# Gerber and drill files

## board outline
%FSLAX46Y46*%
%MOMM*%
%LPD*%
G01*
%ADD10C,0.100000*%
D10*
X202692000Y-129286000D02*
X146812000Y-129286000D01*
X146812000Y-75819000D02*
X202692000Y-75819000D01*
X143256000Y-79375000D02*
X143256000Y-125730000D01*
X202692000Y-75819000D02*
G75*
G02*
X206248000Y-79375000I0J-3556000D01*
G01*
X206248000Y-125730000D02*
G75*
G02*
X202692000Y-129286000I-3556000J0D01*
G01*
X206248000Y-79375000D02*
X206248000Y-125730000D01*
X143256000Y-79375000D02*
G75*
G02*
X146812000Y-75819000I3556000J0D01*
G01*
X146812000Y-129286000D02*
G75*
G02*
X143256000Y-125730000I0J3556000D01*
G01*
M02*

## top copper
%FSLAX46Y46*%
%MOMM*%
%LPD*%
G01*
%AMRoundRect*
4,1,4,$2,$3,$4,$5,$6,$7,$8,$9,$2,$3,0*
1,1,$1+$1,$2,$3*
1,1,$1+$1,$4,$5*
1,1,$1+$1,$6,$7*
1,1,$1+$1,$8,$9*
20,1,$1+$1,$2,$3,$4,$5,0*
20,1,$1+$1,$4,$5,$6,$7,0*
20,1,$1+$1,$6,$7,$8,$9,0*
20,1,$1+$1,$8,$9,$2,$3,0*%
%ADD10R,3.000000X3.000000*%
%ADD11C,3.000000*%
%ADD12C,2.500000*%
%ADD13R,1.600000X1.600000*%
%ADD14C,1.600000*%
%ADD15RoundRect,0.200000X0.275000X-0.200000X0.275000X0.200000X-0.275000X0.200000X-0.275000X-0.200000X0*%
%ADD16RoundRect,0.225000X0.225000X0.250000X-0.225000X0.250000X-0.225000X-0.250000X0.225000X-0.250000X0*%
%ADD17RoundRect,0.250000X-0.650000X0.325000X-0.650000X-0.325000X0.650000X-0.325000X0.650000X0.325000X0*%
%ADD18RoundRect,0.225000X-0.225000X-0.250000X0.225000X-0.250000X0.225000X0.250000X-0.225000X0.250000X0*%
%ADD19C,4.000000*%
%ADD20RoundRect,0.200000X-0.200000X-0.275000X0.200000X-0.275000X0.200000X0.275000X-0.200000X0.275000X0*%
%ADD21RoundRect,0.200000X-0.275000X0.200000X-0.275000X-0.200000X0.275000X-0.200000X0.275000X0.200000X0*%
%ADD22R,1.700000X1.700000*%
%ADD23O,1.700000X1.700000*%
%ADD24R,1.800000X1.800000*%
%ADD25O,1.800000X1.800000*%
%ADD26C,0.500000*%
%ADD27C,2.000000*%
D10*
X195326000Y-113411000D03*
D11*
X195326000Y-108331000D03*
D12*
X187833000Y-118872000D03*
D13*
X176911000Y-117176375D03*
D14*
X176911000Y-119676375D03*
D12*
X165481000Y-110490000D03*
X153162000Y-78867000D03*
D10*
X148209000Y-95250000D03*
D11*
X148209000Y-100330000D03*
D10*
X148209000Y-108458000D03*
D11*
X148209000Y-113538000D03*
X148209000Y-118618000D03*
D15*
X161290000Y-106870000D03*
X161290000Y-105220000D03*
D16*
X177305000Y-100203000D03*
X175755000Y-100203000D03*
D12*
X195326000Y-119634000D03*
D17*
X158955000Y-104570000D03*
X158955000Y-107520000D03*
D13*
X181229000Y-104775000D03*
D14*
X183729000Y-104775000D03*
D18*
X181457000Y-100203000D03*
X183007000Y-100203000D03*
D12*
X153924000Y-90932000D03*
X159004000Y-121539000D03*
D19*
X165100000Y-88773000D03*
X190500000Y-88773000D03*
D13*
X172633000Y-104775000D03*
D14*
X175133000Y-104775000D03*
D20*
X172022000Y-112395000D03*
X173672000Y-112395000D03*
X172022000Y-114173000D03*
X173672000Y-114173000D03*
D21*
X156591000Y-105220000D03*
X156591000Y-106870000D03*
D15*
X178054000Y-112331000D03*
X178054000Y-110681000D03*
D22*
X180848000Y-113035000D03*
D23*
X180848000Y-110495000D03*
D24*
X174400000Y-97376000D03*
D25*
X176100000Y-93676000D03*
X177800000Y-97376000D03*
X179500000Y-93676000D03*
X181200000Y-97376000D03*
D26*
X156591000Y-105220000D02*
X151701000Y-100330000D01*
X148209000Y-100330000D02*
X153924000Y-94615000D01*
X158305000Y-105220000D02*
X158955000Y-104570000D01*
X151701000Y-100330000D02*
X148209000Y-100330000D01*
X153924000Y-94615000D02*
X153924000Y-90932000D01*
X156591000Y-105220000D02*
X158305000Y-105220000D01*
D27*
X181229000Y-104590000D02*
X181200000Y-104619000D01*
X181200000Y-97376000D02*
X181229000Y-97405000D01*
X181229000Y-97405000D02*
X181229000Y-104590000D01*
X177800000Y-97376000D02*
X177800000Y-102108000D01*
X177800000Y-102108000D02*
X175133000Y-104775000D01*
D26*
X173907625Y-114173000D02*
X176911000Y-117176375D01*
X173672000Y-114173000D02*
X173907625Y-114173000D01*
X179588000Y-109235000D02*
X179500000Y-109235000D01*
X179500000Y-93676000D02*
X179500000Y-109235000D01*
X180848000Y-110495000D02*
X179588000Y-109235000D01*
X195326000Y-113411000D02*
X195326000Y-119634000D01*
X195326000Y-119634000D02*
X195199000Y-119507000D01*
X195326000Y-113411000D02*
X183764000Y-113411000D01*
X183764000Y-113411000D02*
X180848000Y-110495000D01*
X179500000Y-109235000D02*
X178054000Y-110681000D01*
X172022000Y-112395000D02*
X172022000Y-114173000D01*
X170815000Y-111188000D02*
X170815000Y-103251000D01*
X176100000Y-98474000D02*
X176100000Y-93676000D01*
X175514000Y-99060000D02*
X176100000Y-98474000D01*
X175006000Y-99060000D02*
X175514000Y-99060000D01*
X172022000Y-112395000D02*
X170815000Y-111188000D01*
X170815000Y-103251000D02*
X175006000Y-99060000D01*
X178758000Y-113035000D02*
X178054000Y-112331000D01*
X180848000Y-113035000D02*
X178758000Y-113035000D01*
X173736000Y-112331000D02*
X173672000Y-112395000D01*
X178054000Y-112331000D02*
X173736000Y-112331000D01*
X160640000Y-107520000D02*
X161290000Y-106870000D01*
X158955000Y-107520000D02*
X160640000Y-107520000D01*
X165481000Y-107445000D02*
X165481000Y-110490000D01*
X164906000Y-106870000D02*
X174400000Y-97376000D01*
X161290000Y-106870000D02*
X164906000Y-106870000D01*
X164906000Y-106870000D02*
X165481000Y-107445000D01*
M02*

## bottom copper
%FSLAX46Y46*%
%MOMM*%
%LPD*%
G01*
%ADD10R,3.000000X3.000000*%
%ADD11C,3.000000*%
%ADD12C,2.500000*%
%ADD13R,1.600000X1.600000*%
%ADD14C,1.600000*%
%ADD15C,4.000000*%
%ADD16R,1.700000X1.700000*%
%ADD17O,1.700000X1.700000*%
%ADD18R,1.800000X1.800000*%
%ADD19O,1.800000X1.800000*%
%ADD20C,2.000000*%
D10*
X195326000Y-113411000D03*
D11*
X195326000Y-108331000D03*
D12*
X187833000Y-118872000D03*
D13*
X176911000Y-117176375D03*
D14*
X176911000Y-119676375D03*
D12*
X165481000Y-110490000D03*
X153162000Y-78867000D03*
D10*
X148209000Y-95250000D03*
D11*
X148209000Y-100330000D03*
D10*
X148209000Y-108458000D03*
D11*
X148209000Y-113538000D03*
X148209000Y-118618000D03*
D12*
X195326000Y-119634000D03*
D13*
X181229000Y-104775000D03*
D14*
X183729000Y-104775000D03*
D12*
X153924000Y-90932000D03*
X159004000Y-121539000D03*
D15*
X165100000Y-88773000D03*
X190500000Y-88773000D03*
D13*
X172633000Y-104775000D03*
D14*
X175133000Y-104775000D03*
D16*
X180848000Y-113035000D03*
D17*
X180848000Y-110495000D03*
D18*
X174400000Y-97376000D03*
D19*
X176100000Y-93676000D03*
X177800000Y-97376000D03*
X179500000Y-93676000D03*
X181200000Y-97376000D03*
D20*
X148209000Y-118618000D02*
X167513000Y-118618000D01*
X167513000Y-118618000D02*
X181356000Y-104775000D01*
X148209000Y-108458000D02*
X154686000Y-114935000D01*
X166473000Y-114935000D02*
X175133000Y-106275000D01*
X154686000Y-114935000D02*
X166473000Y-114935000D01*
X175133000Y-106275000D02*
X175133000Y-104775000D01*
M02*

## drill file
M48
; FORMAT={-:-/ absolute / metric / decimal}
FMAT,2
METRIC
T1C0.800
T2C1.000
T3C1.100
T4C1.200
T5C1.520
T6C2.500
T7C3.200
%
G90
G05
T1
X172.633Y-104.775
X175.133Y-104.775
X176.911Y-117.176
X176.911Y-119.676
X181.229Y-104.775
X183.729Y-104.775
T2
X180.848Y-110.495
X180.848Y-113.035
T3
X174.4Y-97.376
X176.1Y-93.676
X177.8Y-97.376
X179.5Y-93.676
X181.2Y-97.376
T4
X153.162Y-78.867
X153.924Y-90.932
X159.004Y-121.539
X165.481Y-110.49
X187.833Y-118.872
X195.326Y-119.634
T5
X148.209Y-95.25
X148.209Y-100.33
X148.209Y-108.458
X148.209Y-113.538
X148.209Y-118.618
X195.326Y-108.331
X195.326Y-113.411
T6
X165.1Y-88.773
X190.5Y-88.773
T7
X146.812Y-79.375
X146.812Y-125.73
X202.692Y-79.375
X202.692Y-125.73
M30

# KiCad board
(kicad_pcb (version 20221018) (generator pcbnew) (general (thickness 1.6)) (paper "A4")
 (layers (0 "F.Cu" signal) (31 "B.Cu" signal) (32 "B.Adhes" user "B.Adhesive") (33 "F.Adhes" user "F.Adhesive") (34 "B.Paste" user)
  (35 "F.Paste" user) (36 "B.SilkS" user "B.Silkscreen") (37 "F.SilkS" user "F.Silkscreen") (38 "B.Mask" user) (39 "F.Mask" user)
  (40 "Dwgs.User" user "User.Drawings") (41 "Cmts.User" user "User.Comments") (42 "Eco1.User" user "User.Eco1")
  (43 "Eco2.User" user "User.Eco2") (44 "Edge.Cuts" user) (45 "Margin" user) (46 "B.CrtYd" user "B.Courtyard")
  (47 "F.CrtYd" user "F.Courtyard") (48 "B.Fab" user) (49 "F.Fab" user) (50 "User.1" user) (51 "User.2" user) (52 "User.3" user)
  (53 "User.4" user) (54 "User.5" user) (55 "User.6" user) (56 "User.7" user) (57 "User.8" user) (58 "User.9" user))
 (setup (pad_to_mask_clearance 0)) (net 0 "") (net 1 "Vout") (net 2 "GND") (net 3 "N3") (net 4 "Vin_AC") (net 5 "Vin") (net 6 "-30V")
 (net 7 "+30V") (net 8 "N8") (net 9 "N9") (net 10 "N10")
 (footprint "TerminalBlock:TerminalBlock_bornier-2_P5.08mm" (layer "F.Cu") (at 195.326 113.411 90)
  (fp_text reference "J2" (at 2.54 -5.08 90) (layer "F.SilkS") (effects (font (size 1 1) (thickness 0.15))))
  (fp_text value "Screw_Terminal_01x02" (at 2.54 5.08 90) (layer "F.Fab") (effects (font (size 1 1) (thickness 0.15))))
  (pad "1" thru_hole rect (at 0 0 90) (size 3 3) (drill 1.52) (layers "*.Cu" "*.Mask") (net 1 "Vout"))
  (pad "2" thru_hole circle (at 5.08 0 90) (size 3 3) (drill 1.52) (layers "*.Cu" "*.Mask") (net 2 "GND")))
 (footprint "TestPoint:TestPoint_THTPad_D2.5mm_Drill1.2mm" (layer "F.Cu") (at 187.833 118.872)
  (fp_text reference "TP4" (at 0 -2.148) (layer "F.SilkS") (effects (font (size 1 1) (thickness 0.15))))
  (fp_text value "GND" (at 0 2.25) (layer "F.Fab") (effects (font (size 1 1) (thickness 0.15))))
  (pad "1" thru_hole circle (at 0 0) (size 2.5 2.5) (drill 1.2) (layers "*.Cu" "*.Mask") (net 2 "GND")))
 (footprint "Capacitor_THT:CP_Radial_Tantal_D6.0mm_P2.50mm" (layer "F.Cu") (at 176.911 117.176375 -90)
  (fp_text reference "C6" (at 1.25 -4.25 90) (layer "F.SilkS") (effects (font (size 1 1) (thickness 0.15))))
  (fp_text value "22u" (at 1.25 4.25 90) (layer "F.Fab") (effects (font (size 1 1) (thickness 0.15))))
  (pad "1" thru_hole rect (at 0 0 270) (size 1.6 1.6) (drill 0.8) (layers "*.Cu" "*.Mask") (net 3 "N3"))
  (pad "2" thru_hole circle (at 2.5 0 270) (size 1.6 1.6) (drill 0.8) (layers "*.Cu" "*.Mask") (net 2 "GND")))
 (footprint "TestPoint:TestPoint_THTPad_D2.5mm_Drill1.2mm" (layer "F.Cu") (at 165.481 110.49)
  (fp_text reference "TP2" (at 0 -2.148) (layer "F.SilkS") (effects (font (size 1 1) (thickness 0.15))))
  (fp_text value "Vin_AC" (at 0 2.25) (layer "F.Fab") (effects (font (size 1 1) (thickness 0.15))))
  (pad "1" thru_hole circle (at 0 0) (size 2.5 2.5) (drill 1.2) (layers "*.Cu" "*.Mask") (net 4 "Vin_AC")))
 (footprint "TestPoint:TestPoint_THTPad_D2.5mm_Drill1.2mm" (layer "F.Cu") (at 153.162 78.867)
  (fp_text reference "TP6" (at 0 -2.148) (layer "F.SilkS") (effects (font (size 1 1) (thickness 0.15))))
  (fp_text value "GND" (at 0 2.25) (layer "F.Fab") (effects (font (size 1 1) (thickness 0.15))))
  (pad "1" thru_hole circle (at 0 0) (size 2.5 2.5) (drill 1.2) (layers "*.Cu" "*.Mask") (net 2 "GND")))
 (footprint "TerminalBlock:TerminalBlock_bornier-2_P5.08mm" (layer "F.Cu") (at 148.209 95.25 -90)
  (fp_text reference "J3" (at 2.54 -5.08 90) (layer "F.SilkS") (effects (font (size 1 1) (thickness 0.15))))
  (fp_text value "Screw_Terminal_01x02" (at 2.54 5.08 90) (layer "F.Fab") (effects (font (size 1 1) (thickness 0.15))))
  (pad "1" thru_hole rect (at 0 0 270) (size 3 3) (drill 1.52) (layers "*.Cu" "*.Mask") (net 2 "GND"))
  (pad "2" thru_hole circle (at 5.08 0 270) (size 3 3) (drill 1.52) (layers "*.Cu" "*.Mask") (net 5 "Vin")))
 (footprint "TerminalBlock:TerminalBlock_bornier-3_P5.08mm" (layer "F.Cu") (at 148.209 108.458 -90)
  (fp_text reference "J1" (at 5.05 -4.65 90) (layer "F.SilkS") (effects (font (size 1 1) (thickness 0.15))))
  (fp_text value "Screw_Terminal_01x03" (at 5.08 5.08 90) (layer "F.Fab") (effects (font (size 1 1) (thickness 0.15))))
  (pad "1" thru_hole rect (at 0 0 270) (size 3 3) (drill 1.52) (layers "*.Cu" "*.Mask") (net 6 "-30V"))
  (pad "2" thru_hole circle (at 5.08 0 270) (size 3 3) (drill 1.52) (layers "*.Cu" "*.Mask") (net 2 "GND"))
  (pad "3" thru_hole circle (at 10.16 0 270) (size 3 3) (drill 1.52) (layers "*.Cu" "*.Mask") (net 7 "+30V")))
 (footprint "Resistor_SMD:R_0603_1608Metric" (layer "F.Cu") (at 161.29 106.045 90)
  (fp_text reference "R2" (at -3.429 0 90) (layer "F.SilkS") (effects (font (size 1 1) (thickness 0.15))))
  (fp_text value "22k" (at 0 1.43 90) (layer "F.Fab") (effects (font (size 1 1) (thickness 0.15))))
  (pad "1" smd roundrect (at -0.825 0 90) (size 0.8 0.95) (layers "F.Cu" "F.Paste" "F.Mask") (roundrect_rratio 0.25) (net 4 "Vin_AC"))
  (pad "2" smd roundrect (at 0.825 0 90) (size 0.8 0.95) (layers "F.Cu" "F.Paste" "F.Mask") (roundrect_rratio 0.25) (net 2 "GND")))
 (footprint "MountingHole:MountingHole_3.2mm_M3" (layer "F.Cu") (at 146.812 79.375)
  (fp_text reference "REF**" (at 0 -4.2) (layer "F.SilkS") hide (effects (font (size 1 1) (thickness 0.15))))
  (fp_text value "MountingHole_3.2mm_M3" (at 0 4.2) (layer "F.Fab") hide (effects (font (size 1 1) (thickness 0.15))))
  (pad "" np_thru_hole circle (at 0 0) (size 3.2 3.2) (drill 3.2) (layers "*.Cu" "*.Mask")))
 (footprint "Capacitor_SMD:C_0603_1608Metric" (layer "F.Cu") (at 176.53 100.203 180)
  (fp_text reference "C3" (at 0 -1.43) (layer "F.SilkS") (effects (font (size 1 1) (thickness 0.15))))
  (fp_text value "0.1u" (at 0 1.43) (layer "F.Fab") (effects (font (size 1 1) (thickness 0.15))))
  (pad "1" smd roundrect (at -0.775 0 180) (size 0.9 0.95) (layers "F.Cu" "F.Paste" "F.Mask") (roundrect_rratio 0.25) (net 6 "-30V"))
  (pad "2" smd roundrect (at 0.775 0 180) (size 0.9 0.95) (layers "F.Cu" "F.Paste" "F.Mask") (roundrect_rratio 0.25) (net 2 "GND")))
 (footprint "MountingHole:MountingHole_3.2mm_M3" (layer "F.Cu") (at 202.692 125.73)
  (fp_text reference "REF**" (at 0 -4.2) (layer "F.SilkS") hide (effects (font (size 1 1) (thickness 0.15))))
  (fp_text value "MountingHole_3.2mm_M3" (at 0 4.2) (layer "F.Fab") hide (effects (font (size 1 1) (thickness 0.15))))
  (pad "" np_thru_hole circle (at 0 0) (size 3.2 3.2) (drill 3.2) (layers "F&B.Cu" "*.Mask")))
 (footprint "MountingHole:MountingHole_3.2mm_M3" (layer "F.Cu") (at 202.692 79.375)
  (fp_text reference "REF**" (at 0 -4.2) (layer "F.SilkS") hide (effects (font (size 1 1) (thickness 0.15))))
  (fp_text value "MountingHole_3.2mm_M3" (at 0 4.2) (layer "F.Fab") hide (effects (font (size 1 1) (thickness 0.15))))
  (pad "" np_thru_hole circle (at 0 0) (size 3.2 3.2) (drill 3.2) (layers "F&B.Cu" "*.Mask")))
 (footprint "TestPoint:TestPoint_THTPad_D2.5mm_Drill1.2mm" (layer "F.Cu") (at 195.326 119.634)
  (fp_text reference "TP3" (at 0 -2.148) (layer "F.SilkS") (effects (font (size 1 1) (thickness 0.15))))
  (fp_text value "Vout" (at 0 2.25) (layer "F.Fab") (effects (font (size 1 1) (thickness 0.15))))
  (pad "1" thru_hole circle (at 0 0) (size 2.5 2.5) (drill 1.2) (layers "*.Cu" "*.Mask") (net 1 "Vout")))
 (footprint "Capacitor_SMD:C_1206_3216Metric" (layer "F.Cu") (at 158.955 106.045 -90)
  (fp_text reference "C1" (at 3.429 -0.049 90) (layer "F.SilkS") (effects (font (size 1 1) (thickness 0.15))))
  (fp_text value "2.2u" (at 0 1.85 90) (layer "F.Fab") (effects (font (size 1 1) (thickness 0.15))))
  (pad "1" smd roundrect (at -1.475 0 270) (size 1.15 1.8) (layers "F.Cu" "F.Paste" "F.Mask") (roundrect_rratio 0.217391) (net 5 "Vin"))
  (pad "2" smd roundrect (at 1.475 0 270) (size 1.15 1.8) (layers "F.Cu" "F.Paste" "F.Mask") (roundrect_rratio 0.217391) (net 4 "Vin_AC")))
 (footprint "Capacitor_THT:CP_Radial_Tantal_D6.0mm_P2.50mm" (layer "F.Cu") (at 181.229 104.775)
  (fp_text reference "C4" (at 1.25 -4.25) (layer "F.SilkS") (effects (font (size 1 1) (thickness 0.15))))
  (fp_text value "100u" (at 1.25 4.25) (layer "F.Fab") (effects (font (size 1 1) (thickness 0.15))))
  (pad "1" thru_hole rect (at 0 0) (size 1.6 1.6) (drill 0.8) (layers "*.Cu" "*.Mask") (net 7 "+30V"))
  (pad "2" thru_hole circle (at 2.5 0) (size 1.6 1.6) (drill 0.8) (layers "*.Cu" "*.Mask") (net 2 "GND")))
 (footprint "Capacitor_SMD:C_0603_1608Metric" (layer "F.Cu") (at 182.232 100.203)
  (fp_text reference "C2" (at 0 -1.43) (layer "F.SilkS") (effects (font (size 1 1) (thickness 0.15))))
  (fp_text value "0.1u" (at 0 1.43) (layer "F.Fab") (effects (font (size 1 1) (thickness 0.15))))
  (pad "1" smd roundrect (at -0.775 0) (size 0.9 0.95) (layers "F.Cu" "F.Paste" "F.Mask") (roundrect_rratio 0.25) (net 7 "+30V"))
  (pad "2" smd roundrect (at 0.775 0) (size 0.9 0.95) (layers "F.Cu" "F.Paste" "F.Mask") (roundrect_rratio 0.25) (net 2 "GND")))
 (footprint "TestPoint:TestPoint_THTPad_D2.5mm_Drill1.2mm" (layer "F.Cu") (at 153.924 90.932)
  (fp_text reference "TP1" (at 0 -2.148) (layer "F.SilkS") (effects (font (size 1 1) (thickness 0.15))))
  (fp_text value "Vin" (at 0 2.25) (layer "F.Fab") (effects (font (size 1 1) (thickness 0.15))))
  (pad "1" thru_hole circle (at 0 0) (size 2.5 2.5) (drill 1.2) (layers "*.Cu" "*.Mask") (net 5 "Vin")))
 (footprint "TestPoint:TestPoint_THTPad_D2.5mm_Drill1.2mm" (layer "F.Cu") (at 159.004 121.539)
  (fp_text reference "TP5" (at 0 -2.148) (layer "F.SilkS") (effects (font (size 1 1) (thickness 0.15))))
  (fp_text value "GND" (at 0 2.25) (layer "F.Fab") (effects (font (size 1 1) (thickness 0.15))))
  (pad "1" thru_hole circle (at 0 0) (size 2.5 2.5) (drill 1.2) (layers "*.Cu" "*.Mask") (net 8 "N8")))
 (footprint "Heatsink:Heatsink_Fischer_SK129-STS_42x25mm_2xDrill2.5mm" (layer "F.Cu") (at 177.8 88.773)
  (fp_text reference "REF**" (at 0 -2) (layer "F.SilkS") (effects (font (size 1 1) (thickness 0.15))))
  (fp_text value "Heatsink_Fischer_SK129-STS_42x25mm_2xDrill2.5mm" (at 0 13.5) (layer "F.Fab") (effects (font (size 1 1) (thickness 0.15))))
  (pad "1" thru_hole circle (at -12.7 0 180) (size 4 4) (drill 2.5) (layers "*.Cu" "*.Mask"))
  (pad "1" thru_hole circle (at 12.7 0) (size 4 4) (drill 2.5) (layers "*.Cu" "*.Mask")))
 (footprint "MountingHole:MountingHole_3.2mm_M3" (layer "F.Cu") (at 146.812 125.73)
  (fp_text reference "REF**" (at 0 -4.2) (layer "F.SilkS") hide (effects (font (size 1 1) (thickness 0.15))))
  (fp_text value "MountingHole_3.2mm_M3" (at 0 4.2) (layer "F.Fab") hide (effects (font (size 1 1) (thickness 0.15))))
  (pad "" np_thru_hole circle (at 0 0) (size 3.2 3.2) (drill 3.2) (layers "F&B.Cu" "*.Mask")))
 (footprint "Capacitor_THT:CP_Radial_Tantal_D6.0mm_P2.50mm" (layer "F.Cu") (at 172.633 104.775)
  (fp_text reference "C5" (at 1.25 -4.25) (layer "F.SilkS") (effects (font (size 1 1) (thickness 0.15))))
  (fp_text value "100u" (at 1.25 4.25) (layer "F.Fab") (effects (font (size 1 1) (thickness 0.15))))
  (pad "1" thru_hole rect (at 0 0) (size 1.6 1.6) (drill 0.8) (layers "*.Cu" "*.Mask") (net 2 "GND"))
  (pad "2" thru_hole circle (at 2.5 0) (size 1.6 1.6) (drill 0.8) (layers "*.Cu" "*.Mask") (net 6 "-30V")))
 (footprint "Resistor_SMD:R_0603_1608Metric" (layer "F.Cu") (at 172.847 112.395)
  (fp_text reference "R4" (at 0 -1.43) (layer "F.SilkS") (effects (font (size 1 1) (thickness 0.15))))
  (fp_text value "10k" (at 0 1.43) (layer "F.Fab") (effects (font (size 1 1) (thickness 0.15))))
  (pad "1" smd roundrect (at -0.825 0) (size 0.8 0.95) (layers "F.Cu" "F.Paste" "F.Mask") (roundrect_rratio 0.25) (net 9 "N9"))
  (pad "2" smd roundrect (at 0.825 0) (size 0.8 0.95) (layers "F.Cu" "F.Paste" "F.Mask") (roundrect_rratio 0.25) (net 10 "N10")))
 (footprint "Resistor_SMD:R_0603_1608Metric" (layer "F.Cu") (at 172.847 114.173)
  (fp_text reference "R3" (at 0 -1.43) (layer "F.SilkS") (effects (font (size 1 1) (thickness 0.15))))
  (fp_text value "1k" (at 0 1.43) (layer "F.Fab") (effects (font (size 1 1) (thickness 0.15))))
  (pad "1" smd roundrect (at -0.825 0) (size 0.8 0.95) (layers "F.Cu" "F.Paste" "F.Mask") (roundrect_rratio 0.25) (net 9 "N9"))
  (pad "2" smd roundrect (at 0.825 0) (size 0.8 0.95) (layers "F.Cu" "F.Paste" "F.Mask") (roundrect_rratio 0.25) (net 3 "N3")))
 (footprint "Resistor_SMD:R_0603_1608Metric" (layer "F.Cu") (at 156.591 106.045 -90)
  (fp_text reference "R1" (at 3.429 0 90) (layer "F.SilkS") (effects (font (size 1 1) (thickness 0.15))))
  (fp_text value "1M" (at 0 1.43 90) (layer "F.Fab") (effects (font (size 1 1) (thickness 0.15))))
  (pad "1" smd roundrect (at -0.825 0 270) (size 0.8 0.95) (layers "F.Cu" "F.Paste" "F.Mask") (roundrect_rratio 0.25) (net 5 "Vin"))
  (pad "2" smd roundrect (at 0.825 0 270) (size 0.8 0.95) (layers "F.Cu" "F.Paste" "F.Mask") (roundrect_rratio 0.25) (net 2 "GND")))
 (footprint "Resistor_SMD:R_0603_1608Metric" (layer "F.Cu") (at 178.054 111.506 90)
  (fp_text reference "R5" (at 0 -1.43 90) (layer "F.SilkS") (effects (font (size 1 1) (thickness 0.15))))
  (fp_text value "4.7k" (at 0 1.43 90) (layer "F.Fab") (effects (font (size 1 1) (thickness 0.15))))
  (pad "1" smd roundrect (at -0.825 0 90) (size 0.8 0.95) (layers "F.Cu" "F.Paste" "F.Mask") (roundrect_rratio 0.25) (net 10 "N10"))
  (pad "2" smd roundrect (at 0.825 0 90) (size 0.8 0.95) (layers "F.Cu" "F.Paste" "F.Mask") (roundrect_rratio 0.25) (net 1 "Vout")))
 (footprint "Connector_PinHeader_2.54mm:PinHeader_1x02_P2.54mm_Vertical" (layer "F.Cu") (at 180.848 113.035 180)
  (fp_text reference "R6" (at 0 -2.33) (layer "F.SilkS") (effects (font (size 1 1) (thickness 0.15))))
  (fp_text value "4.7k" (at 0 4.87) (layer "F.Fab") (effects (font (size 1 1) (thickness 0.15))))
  (pad "1" thru_hole rect (at 0 0 180) (size 1.7 1.7) (drill 1) (layers "*.Cu" "*.Mask") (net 10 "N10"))
  (pad "2" thru_hole oval (at 0 2.54 180) (size 1.7 1.7) (drill 1) (layers "*.Cu" "*.Mask") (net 1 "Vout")))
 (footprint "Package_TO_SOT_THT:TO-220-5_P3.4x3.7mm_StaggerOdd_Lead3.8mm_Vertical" (layer "F.Cu") (at 174.4 97.376)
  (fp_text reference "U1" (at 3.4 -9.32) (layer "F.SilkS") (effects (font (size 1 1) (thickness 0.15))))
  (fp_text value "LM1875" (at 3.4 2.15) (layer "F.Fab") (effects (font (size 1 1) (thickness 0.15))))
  (pad "1" thru_hole rect (at 0 0) (size 1.8 1.8) (drill 1.1) (layers "*.Cu" "*.Mask") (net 4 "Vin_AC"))
  (pad "2" thru_hole oval (at 1.7 -3.7) (size 1.8 1.8) (drill 1.1) (layers "*.Cu" "*.Mask") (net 9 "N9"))
  (pad "3" thru_hole oval (at 3.4 0) (size 1.8 1.8) (drill 1.1) (layers "*.Cu" "*.Mask") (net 6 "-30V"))
  (pad "4" thru_hole oval (at 5.1 -3.7) (size 1.8 1.8) (drill 1.1) (layers "*.Cu" "*.Mask") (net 1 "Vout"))
  (pad "5" thru_hole oval (at 6.8 0) (size 1.8 1.8) (drill 1.1) (layers "*.Cu" "*.Mask") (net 7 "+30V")))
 (gr_line (start 202.692 129.286) (end 146.812 129.286) (stroke (width 0.1) (type default)) (layer "Edge.Cuts"))
 (gr_line (start 146.812 75.819) (end 202.692 75.819) (stroke (width 0.1) (type default)) (layer "Edge.Cuts"))
 (gr_line (start 143.256 79.375) (end 143.256 125.73) (stroke (width 0.1) (type default)) (layer "Edge.Cuts"))
 (gr_arc (start 202.692 75.819) (mid 205.206472 76.860528) (end 206.248 79.375) (stroke (width 0.1) (type default)) (layer "Edge.Cuts"))
 (gr_arc (start 206.248 125.73) (mid 205.206472 128.244472) (end 202.692 129.286) (stroke (width 0.1) (type default)) (layer "Edge.Cuts"))
 (gr_line (start 206.248 79.375) (end 206.248 125.73) (stroke (width 0.1) (type default)) (layer "Edge.Cuts"))
 (gr_arc (start 143.256 79.375) (mid 144.297528 76.860528) (end 146.812 75.819) (stroke (width 0.1) (type default)) (layer "Edge.Cuts"))
 (gr_arc (start 146.812 129.286) (mid 144.297528 128.244472) (end 143.256 125.73) (stroke (width 0.1) (type default)) (layer "Edge.Cuts"))
 (segment (start 156.591 105.22) (end 151.701 100.33) (width 0.5) (layer "F.Cu") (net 5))
 (segment (start 148.209 100.33) (end 153.924 94.615) (width 0.5) (layer "F.Cu") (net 5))
 (segment (start 158.305 105.22) (end 158.955 104.57) (width 0.5) (layer "F.Cu") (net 5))
 (segment (start 151.701 100.33) (end 148.209 100.33) (width 0.5) (layer "F.Cu") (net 5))
 (segment (start 153.924 94.615) (end 153.924 90.932) (width 0.5) (layer "F.Cu") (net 5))
 (segment (start 156.591 105.22) (end 158.305 105.22) (width 0.5) (layer "F.Cu") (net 5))
 (segment (start 181.229 104.59) (end 181.2 104.619) (width 2) (layer "F.Cu") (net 7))
 (segment (start 181.2 97.376) (end 181.229 97.405) (width 2) (layer "F.Cu") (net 7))
 (segment (start 181.229 97.405) (end 181.229 104.59) (width 2) (layer "F.Cu") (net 7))
 (segment (start 148.209 118.618) (end 167.513 118.618) (width 2) (layer "B.Cu") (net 7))
 (segment (start 167.513 118.618) (end 181.356 104.775) (width 2) (layer "B.Cu") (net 7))
 (segment (start 177.8 97.376) (end 177.8 102.108) (width 2) (layer "F.Cu") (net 6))
 (segment (start 177.8 102.108) (end 175.133 104.775) (width 2) (layer "F.Cu") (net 6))
 (segment (start 148.209 108.458) (end 154.686 114.935) (width 2) (layer "B.Cu") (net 6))
 (segment (start 166.473 114.935) (end 175.133 106.275) (width 2) (layer "B.Cu") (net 6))
 (segment (start 154.686 114.935) (end 166.473 114.935) (width 2) (layer "B.Cu") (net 6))
 (segment (start 175.133 106.275) (end 175.133 104.775) (width 2) (layer "B.Cu") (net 6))
 (segment (start 173.907625 114.173) (end 176.911 117.176375) (width 0.5) (layer "F.Cu") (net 3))
 (segment (start 173.672 114.173) (end 173.907625 114.173) (width 0.5) (layer "F.Cu") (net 3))
 (segment (start 179.588 109.235) (end 179.5 109.235) (width 0.5) (layer "F.Cu") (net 1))
 (segment (start 179.5 93.676) (end 179.5 109.235) (width 0.5) (layer "F.Cu") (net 1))
 (segment (start 180.848 110.495) (end 179.588 109.235) (width 0.5) (layer "F.Cu") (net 1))
 (segment (start 195.326 113.411) (end 195.326 119.634) (width 0.5) (layer "F.Cu") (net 1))
 (segment (start 195.326 119.634) (end 195.199 119.507) (width 0.5) (layer "F.Cu") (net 1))
 (segment (start 195.326 113.411) (end 183.764 113.411) (width 0.5) (layer "F.Cu") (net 1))
 (segment (start 183.764 113.411) (end 180.848 110.495) (width 0.5) (layer "F.Cu") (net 1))
 (segment (start 179.5 109.235) (end 178.054 110.681) (width 0.5) (layer "F.Cu") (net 1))
 (segment (start 172.022 112.395) (end 172.022 114.173) (width 0.5) (layer "F.Cu") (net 9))
 (segment (start 170.815 111.188) (end 170.815 103.251) (width 0.5) (layer "F.Cu") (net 9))
 (segment (start 176.1 98.474) (end 176.1 93.676) (width 0.5) (layer "F.Cu") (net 9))
 (segment (start 175.514 99.06) (end 176.1 98.474) (width 0.5) (layer "F.Cu") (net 9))
 (segment (start 175.006 99.06) (end 175.514 99.06) (width 0.5) (layer "F.Cu") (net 9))
 (segment (start 172.022 112.395) (end 170.815 111.188) (width 0.5) (layer "F.Cu") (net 9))
 (segment (start 170.815 103.251) (end 175.006 99.06) (width 0.5) (layer "F.Cu") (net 9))
 (segment (start 178.758 113.035) (end 178.054 112.331) (width 0.5) (layer "F.Cu") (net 10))
 (segment (start 180.848 113.035) (end 178.758 113.035) (width 0.5) (layer "F.Cu") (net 10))
 (segment (start 173.736 112.331) (end 173.672 112.395) (width 0.5) (layer "F.Cu") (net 10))
 (segment (start 178.054 112.331) (end 173.736 112.331) (width 0.5) (layer "F.Cu") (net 10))
 (segment (start 160.64 107.52) (end 161.29 106.87) (width 0.5) (layer "F.Cu") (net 4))
 (segment (start 158.955 107.52) (end 160.64 107.52) (width 0.5) (layer "F.Cu") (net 4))
 (segment (start 165.481 107.445) (end 165.481 110.49) (width 0.5) (layer "F.Cu") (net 4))
 (segment (start 164.906 106.87) (end 174.4 97.376) (width 0.5) (layer "F.Cu") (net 4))
 (segment (start 161.29 106.87) (end 164.906 106.87) (width 0.5) (layer "F.Cu") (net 4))
 (segment (start 164.906 106.87) (end 165.481 107.445) (width 0.5) (layer "F.Cu") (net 4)))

